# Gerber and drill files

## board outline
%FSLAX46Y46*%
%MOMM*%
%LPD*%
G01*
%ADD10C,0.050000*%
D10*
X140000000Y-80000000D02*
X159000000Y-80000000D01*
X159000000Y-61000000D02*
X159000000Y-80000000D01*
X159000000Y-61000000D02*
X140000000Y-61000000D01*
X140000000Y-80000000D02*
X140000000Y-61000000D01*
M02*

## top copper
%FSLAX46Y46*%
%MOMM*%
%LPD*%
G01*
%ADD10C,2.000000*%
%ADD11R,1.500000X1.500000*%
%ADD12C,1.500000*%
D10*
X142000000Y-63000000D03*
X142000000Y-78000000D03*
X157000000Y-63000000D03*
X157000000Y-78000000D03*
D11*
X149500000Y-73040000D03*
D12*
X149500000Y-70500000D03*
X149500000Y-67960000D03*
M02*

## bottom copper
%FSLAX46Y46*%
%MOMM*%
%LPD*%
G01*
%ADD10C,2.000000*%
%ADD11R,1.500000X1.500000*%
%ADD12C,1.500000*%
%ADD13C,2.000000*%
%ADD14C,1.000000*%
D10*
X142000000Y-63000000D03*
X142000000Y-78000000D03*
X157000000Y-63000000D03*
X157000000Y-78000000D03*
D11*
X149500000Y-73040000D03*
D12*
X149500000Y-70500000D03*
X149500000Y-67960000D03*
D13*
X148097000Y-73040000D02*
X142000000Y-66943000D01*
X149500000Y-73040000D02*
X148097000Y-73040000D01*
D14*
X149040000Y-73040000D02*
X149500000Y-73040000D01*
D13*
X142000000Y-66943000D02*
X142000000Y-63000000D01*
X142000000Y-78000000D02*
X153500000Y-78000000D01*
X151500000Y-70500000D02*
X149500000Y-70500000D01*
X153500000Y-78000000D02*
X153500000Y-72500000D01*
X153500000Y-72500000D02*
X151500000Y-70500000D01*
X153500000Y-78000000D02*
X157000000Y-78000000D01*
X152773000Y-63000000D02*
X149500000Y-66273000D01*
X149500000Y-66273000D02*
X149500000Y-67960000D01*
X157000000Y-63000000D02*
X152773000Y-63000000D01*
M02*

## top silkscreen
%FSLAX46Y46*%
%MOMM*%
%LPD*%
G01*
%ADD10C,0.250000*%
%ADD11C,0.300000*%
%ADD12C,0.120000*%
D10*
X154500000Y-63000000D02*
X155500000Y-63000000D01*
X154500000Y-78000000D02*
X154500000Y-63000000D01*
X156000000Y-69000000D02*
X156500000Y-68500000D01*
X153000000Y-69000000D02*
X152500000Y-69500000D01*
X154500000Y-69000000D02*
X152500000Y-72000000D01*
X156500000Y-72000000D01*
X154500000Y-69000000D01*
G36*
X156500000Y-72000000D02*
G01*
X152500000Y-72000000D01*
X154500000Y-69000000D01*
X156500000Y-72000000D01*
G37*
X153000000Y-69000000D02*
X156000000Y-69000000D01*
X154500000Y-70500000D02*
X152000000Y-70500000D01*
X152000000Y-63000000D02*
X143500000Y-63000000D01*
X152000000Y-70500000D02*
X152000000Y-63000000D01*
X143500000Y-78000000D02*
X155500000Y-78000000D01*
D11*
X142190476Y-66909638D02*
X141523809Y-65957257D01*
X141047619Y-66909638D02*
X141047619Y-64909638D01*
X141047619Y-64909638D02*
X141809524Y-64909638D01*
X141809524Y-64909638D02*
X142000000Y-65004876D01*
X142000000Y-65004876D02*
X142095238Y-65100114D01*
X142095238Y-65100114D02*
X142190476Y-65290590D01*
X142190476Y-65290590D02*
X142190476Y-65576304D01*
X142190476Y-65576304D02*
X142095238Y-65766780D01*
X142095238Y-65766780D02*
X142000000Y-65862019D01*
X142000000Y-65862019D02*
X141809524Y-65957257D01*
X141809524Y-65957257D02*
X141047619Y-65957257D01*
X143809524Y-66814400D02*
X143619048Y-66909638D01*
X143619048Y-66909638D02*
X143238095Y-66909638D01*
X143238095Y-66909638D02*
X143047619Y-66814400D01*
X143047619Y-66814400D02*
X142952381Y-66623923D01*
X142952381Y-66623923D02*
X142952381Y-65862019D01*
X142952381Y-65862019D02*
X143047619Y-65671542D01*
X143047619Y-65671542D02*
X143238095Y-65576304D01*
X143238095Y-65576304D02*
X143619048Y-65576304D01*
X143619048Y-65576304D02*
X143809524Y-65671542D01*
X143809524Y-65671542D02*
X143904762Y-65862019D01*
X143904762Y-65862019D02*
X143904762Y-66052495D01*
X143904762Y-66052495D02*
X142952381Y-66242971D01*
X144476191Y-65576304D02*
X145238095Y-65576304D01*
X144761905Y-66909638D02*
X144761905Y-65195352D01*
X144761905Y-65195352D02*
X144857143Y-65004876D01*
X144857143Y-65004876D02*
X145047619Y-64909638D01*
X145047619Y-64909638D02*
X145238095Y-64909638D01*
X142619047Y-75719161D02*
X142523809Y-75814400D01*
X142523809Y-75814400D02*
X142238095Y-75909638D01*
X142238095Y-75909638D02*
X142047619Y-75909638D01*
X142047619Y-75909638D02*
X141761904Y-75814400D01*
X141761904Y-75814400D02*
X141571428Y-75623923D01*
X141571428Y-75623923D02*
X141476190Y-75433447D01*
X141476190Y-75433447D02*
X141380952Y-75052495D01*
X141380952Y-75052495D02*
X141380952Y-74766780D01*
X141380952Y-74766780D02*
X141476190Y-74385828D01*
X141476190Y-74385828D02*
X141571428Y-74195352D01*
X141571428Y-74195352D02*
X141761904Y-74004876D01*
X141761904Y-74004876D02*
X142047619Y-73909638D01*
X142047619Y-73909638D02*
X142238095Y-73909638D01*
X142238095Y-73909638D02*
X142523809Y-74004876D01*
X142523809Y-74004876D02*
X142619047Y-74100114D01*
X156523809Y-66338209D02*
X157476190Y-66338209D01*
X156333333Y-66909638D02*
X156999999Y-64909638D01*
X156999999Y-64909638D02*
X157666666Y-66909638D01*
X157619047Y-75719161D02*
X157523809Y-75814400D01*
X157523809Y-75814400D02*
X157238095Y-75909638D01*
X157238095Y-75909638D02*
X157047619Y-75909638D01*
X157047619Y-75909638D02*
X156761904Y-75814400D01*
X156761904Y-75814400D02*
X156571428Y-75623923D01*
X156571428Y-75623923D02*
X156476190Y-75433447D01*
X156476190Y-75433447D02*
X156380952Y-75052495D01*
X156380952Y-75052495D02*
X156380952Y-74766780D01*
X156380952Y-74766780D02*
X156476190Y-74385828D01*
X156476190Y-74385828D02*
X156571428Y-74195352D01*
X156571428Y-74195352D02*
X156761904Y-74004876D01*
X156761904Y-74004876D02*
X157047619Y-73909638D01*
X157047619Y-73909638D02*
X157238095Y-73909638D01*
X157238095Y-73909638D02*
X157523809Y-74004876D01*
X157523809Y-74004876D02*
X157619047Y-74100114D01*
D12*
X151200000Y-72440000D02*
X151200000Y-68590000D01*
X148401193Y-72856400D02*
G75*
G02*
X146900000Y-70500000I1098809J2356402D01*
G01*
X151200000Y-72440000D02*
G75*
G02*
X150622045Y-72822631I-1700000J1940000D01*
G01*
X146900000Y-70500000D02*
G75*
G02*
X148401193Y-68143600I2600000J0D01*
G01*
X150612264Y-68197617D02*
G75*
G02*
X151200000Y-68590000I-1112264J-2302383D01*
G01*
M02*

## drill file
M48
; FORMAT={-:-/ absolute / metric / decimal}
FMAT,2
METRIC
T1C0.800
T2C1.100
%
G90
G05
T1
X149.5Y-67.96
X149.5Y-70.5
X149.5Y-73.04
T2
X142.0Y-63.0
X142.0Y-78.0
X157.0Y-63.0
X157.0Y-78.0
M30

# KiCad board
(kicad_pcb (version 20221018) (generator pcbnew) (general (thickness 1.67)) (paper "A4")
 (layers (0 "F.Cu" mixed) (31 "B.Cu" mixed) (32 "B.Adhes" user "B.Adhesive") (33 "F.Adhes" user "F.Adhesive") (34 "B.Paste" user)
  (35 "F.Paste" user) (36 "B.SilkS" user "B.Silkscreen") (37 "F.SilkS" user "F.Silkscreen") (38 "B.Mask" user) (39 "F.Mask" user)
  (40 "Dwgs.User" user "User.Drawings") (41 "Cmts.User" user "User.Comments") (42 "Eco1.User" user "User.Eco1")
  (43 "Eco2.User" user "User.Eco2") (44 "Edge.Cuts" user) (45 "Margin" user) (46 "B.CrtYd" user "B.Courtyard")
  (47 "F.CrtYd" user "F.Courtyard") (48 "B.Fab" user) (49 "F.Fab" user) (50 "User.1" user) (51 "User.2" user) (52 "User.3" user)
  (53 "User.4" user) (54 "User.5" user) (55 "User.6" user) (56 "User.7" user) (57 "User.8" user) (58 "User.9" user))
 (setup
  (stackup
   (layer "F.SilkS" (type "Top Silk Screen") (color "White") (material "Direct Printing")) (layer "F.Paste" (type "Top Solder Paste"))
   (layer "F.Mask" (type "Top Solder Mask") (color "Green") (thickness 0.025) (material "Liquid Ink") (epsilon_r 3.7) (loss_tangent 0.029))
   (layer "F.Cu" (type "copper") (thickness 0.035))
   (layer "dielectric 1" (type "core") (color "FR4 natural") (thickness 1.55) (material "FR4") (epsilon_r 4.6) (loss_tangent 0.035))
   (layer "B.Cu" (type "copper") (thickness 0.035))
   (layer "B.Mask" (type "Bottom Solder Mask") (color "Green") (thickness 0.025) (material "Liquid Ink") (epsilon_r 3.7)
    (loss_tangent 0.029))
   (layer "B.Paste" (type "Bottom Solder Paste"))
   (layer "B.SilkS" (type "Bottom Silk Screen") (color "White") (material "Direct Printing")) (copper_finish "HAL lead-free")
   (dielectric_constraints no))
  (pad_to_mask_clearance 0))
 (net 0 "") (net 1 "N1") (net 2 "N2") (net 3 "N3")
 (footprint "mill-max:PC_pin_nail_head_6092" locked (layer "F.Cu") (at 142 63)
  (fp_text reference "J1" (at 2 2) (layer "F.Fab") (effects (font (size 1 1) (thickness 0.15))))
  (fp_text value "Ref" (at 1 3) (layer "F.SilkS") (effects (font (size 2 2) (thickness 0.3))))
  (pad "1" thru_hole circle locked (at 0 0) (size 2 2) (drill 1.1) (layers "*.Cu" "*.Mask") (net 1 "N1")))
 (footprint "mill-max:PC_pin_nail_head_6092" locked (layer "F.Cu") (at 142 78)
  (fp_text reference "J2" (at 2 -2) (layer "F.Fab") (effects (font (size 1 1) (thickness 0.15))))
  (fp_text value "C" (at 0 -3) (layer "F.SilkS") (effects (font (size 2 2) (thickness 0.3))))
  (pad "1" thru_hole circle locked (at 0 0) (size 2 2) (drill 1.1) (layers "*.Cu" "*.Mask") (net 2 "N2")))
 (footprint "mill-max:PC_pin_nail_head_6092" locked (layer "F.Cu") (at 157 63)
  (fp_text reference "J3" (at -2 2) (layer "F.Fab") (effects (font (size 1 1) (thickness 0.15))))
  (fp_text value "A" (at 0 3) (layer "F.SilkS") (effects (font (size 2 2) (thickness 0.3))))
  (pad "1" thru_hole circle locked (at 0 0) (size 2 2) (drill 1.1) (layers "*.Cu" "*.Mask") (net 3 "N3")))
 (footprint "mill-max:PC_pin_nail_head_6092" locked (layer "F.Cu") (at 157 78)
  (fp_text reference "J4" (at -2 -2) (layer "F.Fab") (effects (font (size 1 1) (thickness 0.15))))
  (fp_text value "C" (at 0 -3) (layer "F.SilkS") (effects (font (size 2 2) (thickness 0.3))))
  (pad "1" thru_hole circle locked (at 0 0) (size 2 2) (drill 1.1) (layers "*.Cu" "*.Mask") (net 2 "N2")))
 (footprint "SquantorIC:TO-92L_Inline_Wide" (layer "F.Cu") (at 149.5 70.5 90)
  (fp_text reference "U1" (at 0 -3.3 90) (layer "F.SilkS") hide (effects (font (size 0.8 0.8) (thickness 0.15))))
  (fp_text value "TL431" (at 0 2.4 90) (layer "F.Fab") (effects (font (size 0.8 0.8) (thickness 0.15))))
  (fp_line (start -1.94 1.7) (end 1.91 1.7) (stroke (width 0.12) (type solid)) (layer "F.SilkS"))
  (fp_arc (start -2.3564 -1.098807) (mid -1.396979 -2.192817) (end 0 -2.6) (stroke (width 0.12) (type solid)) (layer "F.SilkS"))
  (fp_arc (start -1.94 1.7) (mid -2.150817 1.423933) (end -2.322631 1.122045) (stroke (width 0.12) (type solid)) (layer "F.SilkS"))
  (fp_arc (start 0 -2.6) (mid 1.396979 -2.192818) (end 2.3564 -1.098807) (stroke (width 0.12) (type solid)) (layer "F.SilkS"))
  (fp_arc (start 2.302383 1.112264) (mid 2.126594 1.419753) (end 1.91 1.7) (stroke (width 0.12) (type solid)) (layer "F.SilkS"))
  (pad "1" thru_hole rect (at -2.54 0 90) (size 1.5 1.5) (drill 0.8) (layers "*.Cu" "*.Mask") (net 1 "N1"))
  (pad "2" thru_hole circle (at 0 0 90) (size 1.5 1.5) (drill 0.8) (layers "*.Cu" "*.Mask") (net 2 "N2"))
  (pad "3" thru_hole circle (at 2.54 0 90) (size 1.5 1.5) (drill 0.8) (layers "*.Cu" "*.Mask") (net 3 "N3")))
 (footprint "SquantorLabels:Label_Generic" (layer "B.Cu") (at 141.1 69.4 -90)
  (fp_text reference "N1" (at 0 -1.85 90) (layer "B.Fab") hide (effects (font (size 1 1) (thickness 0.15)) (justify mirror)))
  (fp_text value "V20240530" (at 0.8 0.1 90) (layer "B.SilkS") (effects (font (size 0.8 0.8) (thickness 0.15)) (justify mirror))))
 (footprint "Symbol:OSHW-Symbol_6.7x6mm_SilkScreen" (layer "B.Cu") (at 145 70 90)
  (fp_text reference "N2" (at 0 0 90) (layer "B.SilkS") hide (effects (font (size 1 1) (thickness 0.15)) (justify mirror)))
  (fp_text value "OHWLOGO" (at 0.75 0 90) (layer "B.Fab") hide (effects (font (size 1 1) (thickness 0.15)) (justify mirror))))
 (gr_line (start 154.5 63) (end 155.5 63) (stroke (width 0.25) (type default)) (layer "F.SilkS"))
 (gr_line (start 154.5 78) (end 154.5 63) (stroke (width 0.25) (type default)) (layer "F.SilkS"))
 (gr_line (start 156 69) (end 156.5 68.5) (stroke (width 0.25) (type default)) (layer "F.SilkS"))
 (gr_line (start 153 69) (end 152.5 69.5) (stroke (width 0.25) (type default)) (layer "F.SilkS"))
 (gr_poly (pts (xy 154.5 69) (xy 152.5 72) (xy 156.5 72)) (stroke (width 0.25) (type solid)) (fill solid) (layer "F.SilkS"))
 (gr_line (start 153 69) (end 156 69) (stroke (width 0.25) (type default)) (layer "F.SilkS"))
 (gr_line (start 154.5 70.5) (end 152 70.5) (stroke (width 0.25) (type default)) (layer "F.SilkS"))
 (gr_line (start 152 63) (end 143.5 63) (stroke (width 0.25) (type default)) (layer "F.SilkS"))
 (gr_line (start 152 70.5) (end 152 63) (stroke (width 0.25) (type default)) (layer "F.SilkS"))
 (gr_line (start 143.5 78) (end 155.5 78) (stroke (width 0.25) (type default)) (layer "F.SilkS"))
 (gr_line (start 140 80) (end 159 80) (stroke (width 0.05) (type solid)) (layer "Edge.Cuts"))
 (gr_line (start 159 61) (end 159 80) (stroke (width 0.05) (type solid)) (layer "Edge.Cuts"))
 (gr_line (start 159 61) (end 140 61) (stroke (width 0.05) (type solid)) (layer "Edge.Cuts"))
 (gr_line (start 140 80) (end 140 61) (stroke (width 0.05) (type solid)) (layer "Edge.Cuts"))
 (segment (start 148.097 73.04) (end 142 66.943) (width 2) (layer "B.Cu") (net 1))
 (segment (start 149.5 73.04) (end 148.097 73.04) (width 2) (layer "B.Cu") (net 1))
 (segment (start 149.04 73.04) (end 149.5 73.04) (width 1) (layer "B.Cu") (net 1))
 (segment (start 142 66.943) (end 142 63) (width 2) (layer "B.Cu") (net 1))
 (segment (start 142 78) (end 153.5 78) (width 2) (layer "B.Cu") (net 2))
 (segment (start 151.5 70.5) (end 149.5 70.5) (width 2) (layer "B.Cu") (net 2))
 (segment (start 153.5 78) (end 153.5 72.5) (width 2) (layer "B.Cu") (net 2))
 (segment (start 153.5 72.5) (end 151.5 70.5) (width 2) (layer "B.Cu") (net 2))
 (segment (start 153.5 78) (end 157 78) (width 2) (layer "B.Cu") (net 2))
 (segment (start 152.773 63) (end 149.5 66.273) (width 2) (layer "B.Cu") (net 3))
 (segment (start 149.5 66.273) (end 149.5 67.96) (width 2) (layer "B.Cu") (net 3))
 (segment (start 157 63) (end 152.773 63) (width 2) (layer "B.Cu") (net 3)))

